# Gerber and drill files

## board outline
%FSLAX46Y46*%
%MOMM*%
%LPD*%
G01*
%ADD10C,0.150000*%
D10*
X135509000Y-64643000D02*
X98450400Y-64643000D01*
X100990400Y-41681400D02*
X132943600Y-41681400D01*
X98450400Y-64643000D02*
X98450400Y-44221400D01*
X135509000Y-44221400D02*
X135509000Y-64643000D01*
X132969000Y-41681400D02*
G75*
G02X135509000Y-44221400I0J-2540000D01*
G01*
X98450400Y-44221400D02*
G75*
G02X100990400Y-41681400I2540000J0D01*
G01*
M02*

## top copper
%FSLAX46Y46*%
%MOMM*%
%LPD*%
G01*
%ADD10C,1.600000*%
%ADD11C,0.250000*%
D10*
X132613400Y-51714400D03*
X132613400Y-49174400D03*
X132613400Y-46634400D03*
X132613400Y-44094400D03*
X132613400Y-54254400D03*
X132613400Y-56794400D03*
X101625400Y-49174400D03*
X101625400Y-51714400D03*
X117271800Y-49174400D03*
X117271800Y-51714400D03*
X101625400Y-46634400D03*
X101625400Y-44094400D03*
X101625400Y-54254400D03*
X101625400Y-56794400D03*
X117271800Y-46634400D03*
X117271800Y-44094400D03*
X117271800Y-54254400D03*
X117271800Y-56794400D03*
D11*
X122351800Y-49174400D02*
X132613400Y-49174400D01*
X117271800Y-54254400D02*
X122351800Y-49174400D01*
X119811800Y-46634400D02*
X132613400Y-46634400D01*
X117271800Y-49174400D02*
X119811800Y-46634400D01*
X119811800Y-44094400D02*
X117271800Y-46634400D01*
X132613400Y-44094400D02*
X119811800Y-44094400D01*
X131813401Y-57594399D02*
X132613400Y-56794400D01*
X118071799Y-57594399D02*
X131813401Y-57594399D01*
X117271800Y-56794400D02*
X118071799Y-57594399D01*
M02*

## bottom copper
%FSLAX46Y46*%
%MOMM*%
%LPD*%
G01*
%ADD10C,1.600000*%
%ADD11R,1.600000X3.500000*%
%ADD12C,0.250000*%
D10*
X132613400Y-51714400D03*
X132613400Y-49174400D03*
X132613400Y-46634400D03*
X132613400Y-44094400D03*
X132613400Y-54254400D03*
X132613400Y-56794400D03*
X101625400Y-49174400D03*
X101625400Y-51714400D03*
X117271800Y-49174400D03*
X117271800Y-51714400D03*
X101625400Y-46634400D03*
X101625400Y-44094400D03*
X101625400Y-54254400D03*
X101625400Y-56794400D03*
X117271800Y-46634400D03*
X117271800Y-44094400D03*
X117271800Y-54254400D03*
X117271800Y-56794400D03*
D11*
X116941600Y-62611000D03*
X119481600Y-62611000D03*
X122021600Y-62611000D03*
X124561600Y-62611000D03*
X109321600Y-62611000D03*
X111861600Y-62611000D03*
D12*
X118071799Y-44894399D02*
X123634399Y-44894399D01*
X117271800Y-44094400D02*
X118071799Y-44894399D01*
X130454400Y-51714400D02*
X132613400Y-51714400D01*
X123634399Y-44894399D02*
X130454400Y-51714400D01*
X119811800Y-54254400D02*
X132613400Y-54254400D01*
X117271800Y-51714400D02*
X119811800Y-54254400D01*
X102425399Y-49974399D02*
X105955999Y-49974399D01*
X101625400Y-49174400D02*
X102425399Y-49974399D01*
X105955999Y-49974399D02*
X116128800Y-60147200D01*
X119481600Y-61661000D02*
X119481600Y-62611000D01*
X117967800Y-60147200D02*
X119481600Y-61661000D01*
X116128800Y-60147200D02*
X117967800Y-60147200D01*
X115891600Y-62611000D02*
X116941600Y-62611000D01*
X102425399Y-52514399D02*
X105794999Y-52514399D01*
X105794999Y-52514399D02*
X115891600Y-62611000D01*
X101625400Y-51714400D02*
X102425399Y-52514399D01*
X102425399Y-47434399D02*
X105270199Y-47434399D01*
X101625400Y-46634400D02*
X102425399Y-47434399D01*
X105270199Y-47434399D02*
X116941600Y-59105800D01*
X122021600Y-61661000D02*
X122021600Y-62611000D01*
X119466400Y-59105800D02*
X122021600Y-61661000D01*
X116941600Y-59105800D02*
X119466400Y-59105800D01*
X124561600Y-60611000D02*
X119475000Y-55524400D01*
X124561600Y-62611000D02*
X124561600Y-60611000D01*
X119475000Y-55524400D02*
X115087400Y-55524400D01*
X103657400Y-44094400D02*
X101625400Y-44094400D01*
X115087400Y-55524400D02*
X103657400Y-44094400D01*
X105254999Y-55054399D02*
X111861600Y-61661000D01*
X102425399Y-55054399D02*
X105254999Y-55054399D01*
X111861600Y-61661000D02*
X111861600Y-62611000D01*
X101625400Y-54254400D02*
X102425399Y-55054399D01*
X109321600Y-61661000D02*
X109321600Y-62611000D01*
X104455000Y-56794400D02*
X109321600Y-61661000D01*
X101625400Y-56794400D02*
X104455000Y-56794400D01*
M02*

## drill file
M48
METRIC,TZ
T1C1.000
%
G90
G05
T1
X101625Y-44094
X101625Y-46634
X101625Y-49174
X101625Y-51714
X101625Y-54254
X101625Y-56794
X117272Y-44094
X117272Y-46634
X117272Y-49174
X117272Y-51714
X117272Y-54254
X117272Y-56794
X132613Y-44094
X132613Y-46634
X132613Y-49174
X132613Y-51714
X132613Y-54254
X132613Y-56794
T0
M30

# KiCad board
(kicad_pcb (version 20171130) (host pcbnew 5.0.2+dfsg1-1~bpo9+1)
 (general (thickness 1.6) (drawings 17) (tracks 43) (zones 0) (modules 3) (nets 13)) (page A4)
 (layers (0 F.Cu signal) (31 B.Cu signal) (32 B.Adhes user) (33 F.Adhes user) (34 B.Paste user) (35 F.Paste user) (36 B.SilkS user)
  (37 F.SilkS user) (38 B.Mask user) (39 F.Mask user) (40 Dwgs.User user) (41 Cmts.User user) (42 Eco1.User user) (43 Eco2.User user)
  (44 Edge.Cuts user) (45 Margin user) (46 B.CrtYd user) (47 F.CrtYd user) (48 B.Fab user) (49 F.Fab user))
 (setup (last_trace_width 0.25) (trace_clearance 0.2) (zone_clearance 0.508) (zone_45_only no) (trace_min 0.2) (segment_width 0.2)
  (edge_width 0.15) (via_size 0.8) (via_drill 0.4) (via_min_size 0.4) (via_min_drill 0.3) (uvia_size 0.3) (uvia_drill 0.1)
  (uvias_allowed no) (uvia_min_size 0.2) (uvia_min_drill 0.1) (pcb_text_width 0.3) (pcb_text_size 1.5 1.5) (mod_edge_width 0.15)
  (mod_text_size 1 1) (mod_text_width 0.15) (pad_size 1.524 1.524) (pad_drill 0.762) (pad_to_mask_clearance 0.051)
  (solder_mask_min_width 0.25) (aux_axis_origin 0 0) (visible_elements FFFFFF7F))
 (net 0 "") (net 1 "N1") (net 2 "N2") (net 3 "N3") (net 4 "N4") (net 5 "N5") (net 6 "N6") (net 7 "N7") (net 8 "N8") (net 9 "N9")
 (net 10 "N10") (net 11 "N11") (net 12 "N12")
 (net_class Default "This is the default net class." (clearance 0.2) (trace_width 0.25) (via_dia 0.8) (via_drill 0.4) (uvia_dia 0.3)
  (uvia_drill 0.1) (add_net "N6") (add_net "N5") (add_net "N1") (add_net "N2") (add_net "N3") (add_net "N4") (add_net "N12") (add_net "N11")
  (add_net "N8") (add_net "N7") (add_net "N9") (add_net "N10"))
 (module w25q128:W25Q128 (layer F.Cu) (at 132.6134 50.4444 90)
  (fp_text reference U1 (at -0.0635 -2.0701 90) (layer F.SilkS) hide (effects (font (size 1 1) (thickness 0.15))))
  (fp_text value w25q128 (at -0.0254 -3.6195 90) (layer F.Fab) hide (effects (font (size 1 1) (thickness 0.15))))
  (pad 3 thru_hole circle (at -1.27 0 90) (size 1.6 1.6) (drill 1) (layers *.Cu *.Mask) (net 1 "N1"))
  (pad 4 thru_hole circle (at 1.27 0 90) (size 1.6 1.6) (drill 1) (layers *.Cu *.Mask) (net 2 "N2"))
  (pad 5 thru_hole circle (at 3.81 0 90) (size 1.6 1.6) (drill 1) (layers *.Cu *.Mask) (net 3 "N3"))
  (pad 6 thru_hole circle (at 6.35 0 90) (size 1.6 1.6) (drill 1) (layers *.Cu *.Mask) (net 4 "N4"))
  (pad 2 thru_hole circle (at -3.81 0 90) (size 1.6 1.6) (drill 1) (layers *.Cu *.Mask) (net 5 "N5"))
  (pad 1 thru_hole circle (at -6.35 0 90) (size 1.6 1.6) (drill 1) (layers *.Cu *.Mask) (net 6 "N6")))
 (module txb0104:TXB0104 (layer F.Cu) (at 109.4486 50.4444)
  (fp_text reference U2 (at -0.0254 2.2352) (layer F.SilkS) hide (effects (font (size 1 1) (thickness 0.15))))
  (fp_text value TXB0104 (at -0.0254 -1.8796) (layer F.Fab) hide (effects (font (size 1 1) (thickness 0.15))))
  (pad 4 thru_hole circle (at -7.8232 -1.27) (size 1.6 1.6) (drill 1) (layers *.Cu *.Mask) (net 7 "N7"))
  (pad 3 thru_hole circle (at -7.8232 1.27) (size 1.6 1.6) (drill 1) (layers *.Cu *.Mask) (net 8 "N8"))
  (pad 10 thru_hole circle (at 7.8232 -1.27) (size 1.6 1.6) (drill 1) (layers *.Cu *.Mask) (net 3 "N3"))
  (pad 9 thru_hole circle (at 7.8232 1.27) (size 1.6 1.6) (drill 1) (layers *.Cu *.Mask) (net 5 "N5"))
  (pad 5 thru_hole circle (at -7.8232 -3.81) (size 1.6 1.6) (drill 1) (layers *.Cu *.Mask) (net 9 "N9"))
  (pad 6 thru_hole circle (at -7.8232 -6.35) (size 1.6 1.6) (drill 1) (layers *.Cu *.Mask) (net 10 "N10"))
  (pad 2 thru_hole circle (at -7.8232 3.81) (size 1.6 1.6) (drill 1) (layers *.Cu *.Mask) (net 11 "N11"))
  (pad 1 thru_hole circle (at -7.8232 6.35) (size 1.6 1.6) (drill 1) (layers *.Cu *.Mask) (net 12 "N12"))
  (pad 11 thru_hole circle (at 7.8232 -3.81) (size 1.6 1.6) (drill 1) (layers *.Cu *.Mask) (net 4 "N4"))
  (pad 12 thru_hole circle (at 7.8232 -6.35) (size 1.6 1.6) (drill 1) (layers *.Cu *.Mask) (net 1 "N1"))
  (pad 8 thru_hole circle (at 7.8232 3.81) (size 1.6 1.6) (drill 1) (layers *.Cu *.Mask) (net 2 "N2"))
  (pad 7 thru_hole circle (at 7.8232 6.35) (size 1.6 1.6) (drill 1) (layers *.Cu *.Mask) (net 6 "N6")))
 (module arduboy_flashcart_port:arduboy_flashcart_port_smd (layer B.Cu) (at 118.2116 62.611)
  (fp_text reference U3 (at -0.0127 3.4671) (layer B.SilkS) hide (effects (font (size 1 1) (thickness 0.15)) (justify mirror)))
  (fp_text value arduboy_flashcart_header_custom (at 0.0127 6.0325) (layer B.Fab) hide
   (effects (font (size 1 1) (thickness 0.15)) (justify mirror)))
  (pad 3 smd rect (at -1.27 0) (size 1.6 3.5) (layers B.Cu B.Paste B.Mask) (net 8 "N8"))
  (pad 4 smd rect (at 1.27 0) (size 1.6 3.5) (layers B.Cu B.Paste B.Mask) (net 7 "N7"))
  (pad 5 smd rect (at 3.81 0) (size 1.6 3.5) (layers B.Cu B.Paste B.Mask) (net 9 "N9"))
  (pad 6 smd rect (at 6.35 0) (size 1.6 3.5) (layers B.Cu B.Paste B.Mask) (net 10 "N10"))
  (pad 1 smd rect (at -8.89 0) (size 1.6 3.5) (layers B.Cu B.Paste B.Mask) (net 12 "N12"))
  (pad 2 smd rect (at -6.35 0) (size 1.6 3.5) (layers B.Cu B.Paste B.Mask) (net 11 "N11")))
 (gr_line (start 135.509 64.643) (end 98.4504 64.643) (layer Edge.Cuts) (width 0.15))
 (gr_line (start 100.9904 41.6814) (end 132.9436 41.6814) (layer Edge.Cuts) (width 0.15))
 (gr_line (start 98.4504 64.643) (end 98.4504 44.2214) (layer Edge.Cuts) (width 0.15))
 (gr_line (start 135.509 44.2214) (end 135.509 64.643) (layer Edge.Cuts) (width 0.15))
 (gr_arc (start 132.969 44.2214) (end 135.509 44.2214) (angle -90) (layer Edge.Cuts) (width 0.15))
 (gr_arc (start 100.9904 44.2214) (end 100.9904 41.6814) (angle -90) (layer Edge.Cuts) (width 0.15))
 (segment (start 118.071799 44.894399) (end 123.634399 44.894399) (width 0.25) (layer B.Cu) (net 1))
 (segment (start 117.2718 44.0944) (end 118.071799 44.894399) (width 0.25) (layer B.Cu) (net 1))
 (segment (start 130.4544 51.7144) (end 132.6134 51.7144) (width 0.25) (layer B.Cu) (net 1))
 (segment (start 123.634399 44.894399) (end 130.4544 51.7144) (width 0.25) (layer B.Cu) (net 1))
 (segment (start 122.3518 49.1744) (end 132.6134 49.1744) (width 0.25) (layer F.Cu) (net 2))
 (segment (start 117.2718 54.2544) (end 122.3518 49.1744) (width 0.25) (layer F.Cu) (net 2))
 (segment (start 119.8118 46.6344) (end 132.6134 46.6344) (width 0.25) (layer F.Cu) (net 3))
 (segment (start 117.2718 49.1744) (end 119.8118 46.6344) (width 0.25) (layer F.Cu) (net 3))
 (segment (start 119.8118 44.0944) (end 117.2718 46.6344) (width 0.25) (layer F.Cu) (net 4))
 (segment (start 132.6134 44.0944) (end 119.8118 44.0944) (width 0.25) (layer F.Cu) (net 4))
 (segment (start 119.8118 54.2544) (end 132.6134 54.2544) (width 0.25) (layer B.Cu) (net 5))
 (segment (start 117.2718 51.7144) (end 119.8118 54.2544) (width 0.25) (layer B.Cu) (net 5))
 (segment (start 131.813401 57.594399) (end 132.6134 56.7944) (width 0.25) (layer F.Cu) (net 6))
 (segment (start 118.071799 57.594399) (end 131.813401 57.594399) (width 0.25) (layer F.Cu) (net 6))
 (segment (start 117.2718 56.7944) (end 118.071799 57.594399) (width 0.25) (layer F.Cu) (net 6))
 (segment (start 102.425399 49.974399) (end 105.955999 49.974399) (width 0.25) (layer B.Cu) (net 7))
 (segment (start 101.6254 49.1744) (end 102.425399 49.974399) (width 0.25) (layer B.Cu) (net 7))
 (segment (start 105.955999 49.974399) (end 116.1288 60.1472) (width 0.25) (layer B.Cu) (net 7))
 (segment (start 119.4816 61.661) (end 119.4816 62.611) (width 0.25) (layer B.Cu) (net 7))
 (segment (start 117.9678 60.1472) (end 119.4816 61.661) (width 0.25) (layer B.Cu) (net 7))
 (segment (start 116.1288 60.1472) (end 117.9678 60.1472) (width 0.25) (layer B.Cu) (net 7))
 (segment (start 115.8916 62.611) (end 116.9416 62.611) (width 0.25) (layer B.Cu) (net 8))
 (segment (start 102.425399 52.514399) (end 105.794999 52.514399) (width 0.25) (layer B.Cu) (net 8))
 (segment (start 105.794999 52.514399) (end 115.8916 62.611) (width 0.25) (layer B.Cu) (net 8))
 (segment (start 101.6254 51.7144) (end 102.425399 52.514399) (width 0.25) (layer B.Cu) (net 8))
 (segment (start 102.425399 47.434399) (end 105.270199 47.434399) (width 0.25) (layer B.Cu) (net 9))
 (segment (start 101.6254 46.6344) (end 102.425399 47.434399) (width 0.25) (layer B.Cu) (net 9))
 (segment (start 105.270199 47.434399) (end 116.9416 59.1058) (width 0.25) (layer B.Cu) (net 9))
 (segment (start 122.0216 61.661) (end 122.0216 62.611) (width 0.25) (layer B.Cu) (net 9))
 (segment (start 119.4664 59.1058) (end 122.0216 61.661) (width 0.25) (layer B.Cu) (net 9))
 (segment (start 116.9416 59.1058) (end 119.4664 59.1058) (width 0.25) (layer B.Cu) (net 9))
 (segment (start 124.5616 60.611) (end 119.475 55.5244) (width 0.25) (layer B.Cu) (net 10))
 (segment (start 124.5616 62.611) (end 124.5616 60.611) (width 0.25) (layer B.Cu) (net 10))
 (segment (start 119.475 55.5244) (end 115.0874 55.5244) (width 0.25) (layer B.Cu) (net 10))
 (segment (start 103.6574 44.0944) (end 101.6254 44.0944) (width 0.25) (layer B.Cu) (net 10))
 (segment (start 115.0874 55.5244) (end 103.6574 44.0944) (width 0.25) (layer B.Cu) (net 10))
 (segment (start 105.254999 55.054399) (end 111.8616 61.661) (width 0.25) (layer B.Cu) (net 11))
 (segment (start 102.425399 55.054399) (end 105.254999 55.054399) (width 0.25) (layer B.Cu) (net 11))
 (segment (start 111.8616 61.661) (end 111.8616 62.611) (width 0.25) (layer B.Cu) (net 11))
 (segment (start 101.6254 54.2544) (end 102.425399 55.054399) (width 0.25) (layer B.Cu) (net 11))
 (segment (start 109.3216 61.661) (end 109.3216 62.611) (width 0.25) (layer B.Cu) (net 12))
 (segment (start 104.455 56.7944) (end 109.3216 61.661) (width 0.25) (layer B.Cu) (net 12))
 (segment (start 101.6254 56.7944) (end 104.455 56.7944) (width 0.25) (layer B.Cu) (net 12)))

